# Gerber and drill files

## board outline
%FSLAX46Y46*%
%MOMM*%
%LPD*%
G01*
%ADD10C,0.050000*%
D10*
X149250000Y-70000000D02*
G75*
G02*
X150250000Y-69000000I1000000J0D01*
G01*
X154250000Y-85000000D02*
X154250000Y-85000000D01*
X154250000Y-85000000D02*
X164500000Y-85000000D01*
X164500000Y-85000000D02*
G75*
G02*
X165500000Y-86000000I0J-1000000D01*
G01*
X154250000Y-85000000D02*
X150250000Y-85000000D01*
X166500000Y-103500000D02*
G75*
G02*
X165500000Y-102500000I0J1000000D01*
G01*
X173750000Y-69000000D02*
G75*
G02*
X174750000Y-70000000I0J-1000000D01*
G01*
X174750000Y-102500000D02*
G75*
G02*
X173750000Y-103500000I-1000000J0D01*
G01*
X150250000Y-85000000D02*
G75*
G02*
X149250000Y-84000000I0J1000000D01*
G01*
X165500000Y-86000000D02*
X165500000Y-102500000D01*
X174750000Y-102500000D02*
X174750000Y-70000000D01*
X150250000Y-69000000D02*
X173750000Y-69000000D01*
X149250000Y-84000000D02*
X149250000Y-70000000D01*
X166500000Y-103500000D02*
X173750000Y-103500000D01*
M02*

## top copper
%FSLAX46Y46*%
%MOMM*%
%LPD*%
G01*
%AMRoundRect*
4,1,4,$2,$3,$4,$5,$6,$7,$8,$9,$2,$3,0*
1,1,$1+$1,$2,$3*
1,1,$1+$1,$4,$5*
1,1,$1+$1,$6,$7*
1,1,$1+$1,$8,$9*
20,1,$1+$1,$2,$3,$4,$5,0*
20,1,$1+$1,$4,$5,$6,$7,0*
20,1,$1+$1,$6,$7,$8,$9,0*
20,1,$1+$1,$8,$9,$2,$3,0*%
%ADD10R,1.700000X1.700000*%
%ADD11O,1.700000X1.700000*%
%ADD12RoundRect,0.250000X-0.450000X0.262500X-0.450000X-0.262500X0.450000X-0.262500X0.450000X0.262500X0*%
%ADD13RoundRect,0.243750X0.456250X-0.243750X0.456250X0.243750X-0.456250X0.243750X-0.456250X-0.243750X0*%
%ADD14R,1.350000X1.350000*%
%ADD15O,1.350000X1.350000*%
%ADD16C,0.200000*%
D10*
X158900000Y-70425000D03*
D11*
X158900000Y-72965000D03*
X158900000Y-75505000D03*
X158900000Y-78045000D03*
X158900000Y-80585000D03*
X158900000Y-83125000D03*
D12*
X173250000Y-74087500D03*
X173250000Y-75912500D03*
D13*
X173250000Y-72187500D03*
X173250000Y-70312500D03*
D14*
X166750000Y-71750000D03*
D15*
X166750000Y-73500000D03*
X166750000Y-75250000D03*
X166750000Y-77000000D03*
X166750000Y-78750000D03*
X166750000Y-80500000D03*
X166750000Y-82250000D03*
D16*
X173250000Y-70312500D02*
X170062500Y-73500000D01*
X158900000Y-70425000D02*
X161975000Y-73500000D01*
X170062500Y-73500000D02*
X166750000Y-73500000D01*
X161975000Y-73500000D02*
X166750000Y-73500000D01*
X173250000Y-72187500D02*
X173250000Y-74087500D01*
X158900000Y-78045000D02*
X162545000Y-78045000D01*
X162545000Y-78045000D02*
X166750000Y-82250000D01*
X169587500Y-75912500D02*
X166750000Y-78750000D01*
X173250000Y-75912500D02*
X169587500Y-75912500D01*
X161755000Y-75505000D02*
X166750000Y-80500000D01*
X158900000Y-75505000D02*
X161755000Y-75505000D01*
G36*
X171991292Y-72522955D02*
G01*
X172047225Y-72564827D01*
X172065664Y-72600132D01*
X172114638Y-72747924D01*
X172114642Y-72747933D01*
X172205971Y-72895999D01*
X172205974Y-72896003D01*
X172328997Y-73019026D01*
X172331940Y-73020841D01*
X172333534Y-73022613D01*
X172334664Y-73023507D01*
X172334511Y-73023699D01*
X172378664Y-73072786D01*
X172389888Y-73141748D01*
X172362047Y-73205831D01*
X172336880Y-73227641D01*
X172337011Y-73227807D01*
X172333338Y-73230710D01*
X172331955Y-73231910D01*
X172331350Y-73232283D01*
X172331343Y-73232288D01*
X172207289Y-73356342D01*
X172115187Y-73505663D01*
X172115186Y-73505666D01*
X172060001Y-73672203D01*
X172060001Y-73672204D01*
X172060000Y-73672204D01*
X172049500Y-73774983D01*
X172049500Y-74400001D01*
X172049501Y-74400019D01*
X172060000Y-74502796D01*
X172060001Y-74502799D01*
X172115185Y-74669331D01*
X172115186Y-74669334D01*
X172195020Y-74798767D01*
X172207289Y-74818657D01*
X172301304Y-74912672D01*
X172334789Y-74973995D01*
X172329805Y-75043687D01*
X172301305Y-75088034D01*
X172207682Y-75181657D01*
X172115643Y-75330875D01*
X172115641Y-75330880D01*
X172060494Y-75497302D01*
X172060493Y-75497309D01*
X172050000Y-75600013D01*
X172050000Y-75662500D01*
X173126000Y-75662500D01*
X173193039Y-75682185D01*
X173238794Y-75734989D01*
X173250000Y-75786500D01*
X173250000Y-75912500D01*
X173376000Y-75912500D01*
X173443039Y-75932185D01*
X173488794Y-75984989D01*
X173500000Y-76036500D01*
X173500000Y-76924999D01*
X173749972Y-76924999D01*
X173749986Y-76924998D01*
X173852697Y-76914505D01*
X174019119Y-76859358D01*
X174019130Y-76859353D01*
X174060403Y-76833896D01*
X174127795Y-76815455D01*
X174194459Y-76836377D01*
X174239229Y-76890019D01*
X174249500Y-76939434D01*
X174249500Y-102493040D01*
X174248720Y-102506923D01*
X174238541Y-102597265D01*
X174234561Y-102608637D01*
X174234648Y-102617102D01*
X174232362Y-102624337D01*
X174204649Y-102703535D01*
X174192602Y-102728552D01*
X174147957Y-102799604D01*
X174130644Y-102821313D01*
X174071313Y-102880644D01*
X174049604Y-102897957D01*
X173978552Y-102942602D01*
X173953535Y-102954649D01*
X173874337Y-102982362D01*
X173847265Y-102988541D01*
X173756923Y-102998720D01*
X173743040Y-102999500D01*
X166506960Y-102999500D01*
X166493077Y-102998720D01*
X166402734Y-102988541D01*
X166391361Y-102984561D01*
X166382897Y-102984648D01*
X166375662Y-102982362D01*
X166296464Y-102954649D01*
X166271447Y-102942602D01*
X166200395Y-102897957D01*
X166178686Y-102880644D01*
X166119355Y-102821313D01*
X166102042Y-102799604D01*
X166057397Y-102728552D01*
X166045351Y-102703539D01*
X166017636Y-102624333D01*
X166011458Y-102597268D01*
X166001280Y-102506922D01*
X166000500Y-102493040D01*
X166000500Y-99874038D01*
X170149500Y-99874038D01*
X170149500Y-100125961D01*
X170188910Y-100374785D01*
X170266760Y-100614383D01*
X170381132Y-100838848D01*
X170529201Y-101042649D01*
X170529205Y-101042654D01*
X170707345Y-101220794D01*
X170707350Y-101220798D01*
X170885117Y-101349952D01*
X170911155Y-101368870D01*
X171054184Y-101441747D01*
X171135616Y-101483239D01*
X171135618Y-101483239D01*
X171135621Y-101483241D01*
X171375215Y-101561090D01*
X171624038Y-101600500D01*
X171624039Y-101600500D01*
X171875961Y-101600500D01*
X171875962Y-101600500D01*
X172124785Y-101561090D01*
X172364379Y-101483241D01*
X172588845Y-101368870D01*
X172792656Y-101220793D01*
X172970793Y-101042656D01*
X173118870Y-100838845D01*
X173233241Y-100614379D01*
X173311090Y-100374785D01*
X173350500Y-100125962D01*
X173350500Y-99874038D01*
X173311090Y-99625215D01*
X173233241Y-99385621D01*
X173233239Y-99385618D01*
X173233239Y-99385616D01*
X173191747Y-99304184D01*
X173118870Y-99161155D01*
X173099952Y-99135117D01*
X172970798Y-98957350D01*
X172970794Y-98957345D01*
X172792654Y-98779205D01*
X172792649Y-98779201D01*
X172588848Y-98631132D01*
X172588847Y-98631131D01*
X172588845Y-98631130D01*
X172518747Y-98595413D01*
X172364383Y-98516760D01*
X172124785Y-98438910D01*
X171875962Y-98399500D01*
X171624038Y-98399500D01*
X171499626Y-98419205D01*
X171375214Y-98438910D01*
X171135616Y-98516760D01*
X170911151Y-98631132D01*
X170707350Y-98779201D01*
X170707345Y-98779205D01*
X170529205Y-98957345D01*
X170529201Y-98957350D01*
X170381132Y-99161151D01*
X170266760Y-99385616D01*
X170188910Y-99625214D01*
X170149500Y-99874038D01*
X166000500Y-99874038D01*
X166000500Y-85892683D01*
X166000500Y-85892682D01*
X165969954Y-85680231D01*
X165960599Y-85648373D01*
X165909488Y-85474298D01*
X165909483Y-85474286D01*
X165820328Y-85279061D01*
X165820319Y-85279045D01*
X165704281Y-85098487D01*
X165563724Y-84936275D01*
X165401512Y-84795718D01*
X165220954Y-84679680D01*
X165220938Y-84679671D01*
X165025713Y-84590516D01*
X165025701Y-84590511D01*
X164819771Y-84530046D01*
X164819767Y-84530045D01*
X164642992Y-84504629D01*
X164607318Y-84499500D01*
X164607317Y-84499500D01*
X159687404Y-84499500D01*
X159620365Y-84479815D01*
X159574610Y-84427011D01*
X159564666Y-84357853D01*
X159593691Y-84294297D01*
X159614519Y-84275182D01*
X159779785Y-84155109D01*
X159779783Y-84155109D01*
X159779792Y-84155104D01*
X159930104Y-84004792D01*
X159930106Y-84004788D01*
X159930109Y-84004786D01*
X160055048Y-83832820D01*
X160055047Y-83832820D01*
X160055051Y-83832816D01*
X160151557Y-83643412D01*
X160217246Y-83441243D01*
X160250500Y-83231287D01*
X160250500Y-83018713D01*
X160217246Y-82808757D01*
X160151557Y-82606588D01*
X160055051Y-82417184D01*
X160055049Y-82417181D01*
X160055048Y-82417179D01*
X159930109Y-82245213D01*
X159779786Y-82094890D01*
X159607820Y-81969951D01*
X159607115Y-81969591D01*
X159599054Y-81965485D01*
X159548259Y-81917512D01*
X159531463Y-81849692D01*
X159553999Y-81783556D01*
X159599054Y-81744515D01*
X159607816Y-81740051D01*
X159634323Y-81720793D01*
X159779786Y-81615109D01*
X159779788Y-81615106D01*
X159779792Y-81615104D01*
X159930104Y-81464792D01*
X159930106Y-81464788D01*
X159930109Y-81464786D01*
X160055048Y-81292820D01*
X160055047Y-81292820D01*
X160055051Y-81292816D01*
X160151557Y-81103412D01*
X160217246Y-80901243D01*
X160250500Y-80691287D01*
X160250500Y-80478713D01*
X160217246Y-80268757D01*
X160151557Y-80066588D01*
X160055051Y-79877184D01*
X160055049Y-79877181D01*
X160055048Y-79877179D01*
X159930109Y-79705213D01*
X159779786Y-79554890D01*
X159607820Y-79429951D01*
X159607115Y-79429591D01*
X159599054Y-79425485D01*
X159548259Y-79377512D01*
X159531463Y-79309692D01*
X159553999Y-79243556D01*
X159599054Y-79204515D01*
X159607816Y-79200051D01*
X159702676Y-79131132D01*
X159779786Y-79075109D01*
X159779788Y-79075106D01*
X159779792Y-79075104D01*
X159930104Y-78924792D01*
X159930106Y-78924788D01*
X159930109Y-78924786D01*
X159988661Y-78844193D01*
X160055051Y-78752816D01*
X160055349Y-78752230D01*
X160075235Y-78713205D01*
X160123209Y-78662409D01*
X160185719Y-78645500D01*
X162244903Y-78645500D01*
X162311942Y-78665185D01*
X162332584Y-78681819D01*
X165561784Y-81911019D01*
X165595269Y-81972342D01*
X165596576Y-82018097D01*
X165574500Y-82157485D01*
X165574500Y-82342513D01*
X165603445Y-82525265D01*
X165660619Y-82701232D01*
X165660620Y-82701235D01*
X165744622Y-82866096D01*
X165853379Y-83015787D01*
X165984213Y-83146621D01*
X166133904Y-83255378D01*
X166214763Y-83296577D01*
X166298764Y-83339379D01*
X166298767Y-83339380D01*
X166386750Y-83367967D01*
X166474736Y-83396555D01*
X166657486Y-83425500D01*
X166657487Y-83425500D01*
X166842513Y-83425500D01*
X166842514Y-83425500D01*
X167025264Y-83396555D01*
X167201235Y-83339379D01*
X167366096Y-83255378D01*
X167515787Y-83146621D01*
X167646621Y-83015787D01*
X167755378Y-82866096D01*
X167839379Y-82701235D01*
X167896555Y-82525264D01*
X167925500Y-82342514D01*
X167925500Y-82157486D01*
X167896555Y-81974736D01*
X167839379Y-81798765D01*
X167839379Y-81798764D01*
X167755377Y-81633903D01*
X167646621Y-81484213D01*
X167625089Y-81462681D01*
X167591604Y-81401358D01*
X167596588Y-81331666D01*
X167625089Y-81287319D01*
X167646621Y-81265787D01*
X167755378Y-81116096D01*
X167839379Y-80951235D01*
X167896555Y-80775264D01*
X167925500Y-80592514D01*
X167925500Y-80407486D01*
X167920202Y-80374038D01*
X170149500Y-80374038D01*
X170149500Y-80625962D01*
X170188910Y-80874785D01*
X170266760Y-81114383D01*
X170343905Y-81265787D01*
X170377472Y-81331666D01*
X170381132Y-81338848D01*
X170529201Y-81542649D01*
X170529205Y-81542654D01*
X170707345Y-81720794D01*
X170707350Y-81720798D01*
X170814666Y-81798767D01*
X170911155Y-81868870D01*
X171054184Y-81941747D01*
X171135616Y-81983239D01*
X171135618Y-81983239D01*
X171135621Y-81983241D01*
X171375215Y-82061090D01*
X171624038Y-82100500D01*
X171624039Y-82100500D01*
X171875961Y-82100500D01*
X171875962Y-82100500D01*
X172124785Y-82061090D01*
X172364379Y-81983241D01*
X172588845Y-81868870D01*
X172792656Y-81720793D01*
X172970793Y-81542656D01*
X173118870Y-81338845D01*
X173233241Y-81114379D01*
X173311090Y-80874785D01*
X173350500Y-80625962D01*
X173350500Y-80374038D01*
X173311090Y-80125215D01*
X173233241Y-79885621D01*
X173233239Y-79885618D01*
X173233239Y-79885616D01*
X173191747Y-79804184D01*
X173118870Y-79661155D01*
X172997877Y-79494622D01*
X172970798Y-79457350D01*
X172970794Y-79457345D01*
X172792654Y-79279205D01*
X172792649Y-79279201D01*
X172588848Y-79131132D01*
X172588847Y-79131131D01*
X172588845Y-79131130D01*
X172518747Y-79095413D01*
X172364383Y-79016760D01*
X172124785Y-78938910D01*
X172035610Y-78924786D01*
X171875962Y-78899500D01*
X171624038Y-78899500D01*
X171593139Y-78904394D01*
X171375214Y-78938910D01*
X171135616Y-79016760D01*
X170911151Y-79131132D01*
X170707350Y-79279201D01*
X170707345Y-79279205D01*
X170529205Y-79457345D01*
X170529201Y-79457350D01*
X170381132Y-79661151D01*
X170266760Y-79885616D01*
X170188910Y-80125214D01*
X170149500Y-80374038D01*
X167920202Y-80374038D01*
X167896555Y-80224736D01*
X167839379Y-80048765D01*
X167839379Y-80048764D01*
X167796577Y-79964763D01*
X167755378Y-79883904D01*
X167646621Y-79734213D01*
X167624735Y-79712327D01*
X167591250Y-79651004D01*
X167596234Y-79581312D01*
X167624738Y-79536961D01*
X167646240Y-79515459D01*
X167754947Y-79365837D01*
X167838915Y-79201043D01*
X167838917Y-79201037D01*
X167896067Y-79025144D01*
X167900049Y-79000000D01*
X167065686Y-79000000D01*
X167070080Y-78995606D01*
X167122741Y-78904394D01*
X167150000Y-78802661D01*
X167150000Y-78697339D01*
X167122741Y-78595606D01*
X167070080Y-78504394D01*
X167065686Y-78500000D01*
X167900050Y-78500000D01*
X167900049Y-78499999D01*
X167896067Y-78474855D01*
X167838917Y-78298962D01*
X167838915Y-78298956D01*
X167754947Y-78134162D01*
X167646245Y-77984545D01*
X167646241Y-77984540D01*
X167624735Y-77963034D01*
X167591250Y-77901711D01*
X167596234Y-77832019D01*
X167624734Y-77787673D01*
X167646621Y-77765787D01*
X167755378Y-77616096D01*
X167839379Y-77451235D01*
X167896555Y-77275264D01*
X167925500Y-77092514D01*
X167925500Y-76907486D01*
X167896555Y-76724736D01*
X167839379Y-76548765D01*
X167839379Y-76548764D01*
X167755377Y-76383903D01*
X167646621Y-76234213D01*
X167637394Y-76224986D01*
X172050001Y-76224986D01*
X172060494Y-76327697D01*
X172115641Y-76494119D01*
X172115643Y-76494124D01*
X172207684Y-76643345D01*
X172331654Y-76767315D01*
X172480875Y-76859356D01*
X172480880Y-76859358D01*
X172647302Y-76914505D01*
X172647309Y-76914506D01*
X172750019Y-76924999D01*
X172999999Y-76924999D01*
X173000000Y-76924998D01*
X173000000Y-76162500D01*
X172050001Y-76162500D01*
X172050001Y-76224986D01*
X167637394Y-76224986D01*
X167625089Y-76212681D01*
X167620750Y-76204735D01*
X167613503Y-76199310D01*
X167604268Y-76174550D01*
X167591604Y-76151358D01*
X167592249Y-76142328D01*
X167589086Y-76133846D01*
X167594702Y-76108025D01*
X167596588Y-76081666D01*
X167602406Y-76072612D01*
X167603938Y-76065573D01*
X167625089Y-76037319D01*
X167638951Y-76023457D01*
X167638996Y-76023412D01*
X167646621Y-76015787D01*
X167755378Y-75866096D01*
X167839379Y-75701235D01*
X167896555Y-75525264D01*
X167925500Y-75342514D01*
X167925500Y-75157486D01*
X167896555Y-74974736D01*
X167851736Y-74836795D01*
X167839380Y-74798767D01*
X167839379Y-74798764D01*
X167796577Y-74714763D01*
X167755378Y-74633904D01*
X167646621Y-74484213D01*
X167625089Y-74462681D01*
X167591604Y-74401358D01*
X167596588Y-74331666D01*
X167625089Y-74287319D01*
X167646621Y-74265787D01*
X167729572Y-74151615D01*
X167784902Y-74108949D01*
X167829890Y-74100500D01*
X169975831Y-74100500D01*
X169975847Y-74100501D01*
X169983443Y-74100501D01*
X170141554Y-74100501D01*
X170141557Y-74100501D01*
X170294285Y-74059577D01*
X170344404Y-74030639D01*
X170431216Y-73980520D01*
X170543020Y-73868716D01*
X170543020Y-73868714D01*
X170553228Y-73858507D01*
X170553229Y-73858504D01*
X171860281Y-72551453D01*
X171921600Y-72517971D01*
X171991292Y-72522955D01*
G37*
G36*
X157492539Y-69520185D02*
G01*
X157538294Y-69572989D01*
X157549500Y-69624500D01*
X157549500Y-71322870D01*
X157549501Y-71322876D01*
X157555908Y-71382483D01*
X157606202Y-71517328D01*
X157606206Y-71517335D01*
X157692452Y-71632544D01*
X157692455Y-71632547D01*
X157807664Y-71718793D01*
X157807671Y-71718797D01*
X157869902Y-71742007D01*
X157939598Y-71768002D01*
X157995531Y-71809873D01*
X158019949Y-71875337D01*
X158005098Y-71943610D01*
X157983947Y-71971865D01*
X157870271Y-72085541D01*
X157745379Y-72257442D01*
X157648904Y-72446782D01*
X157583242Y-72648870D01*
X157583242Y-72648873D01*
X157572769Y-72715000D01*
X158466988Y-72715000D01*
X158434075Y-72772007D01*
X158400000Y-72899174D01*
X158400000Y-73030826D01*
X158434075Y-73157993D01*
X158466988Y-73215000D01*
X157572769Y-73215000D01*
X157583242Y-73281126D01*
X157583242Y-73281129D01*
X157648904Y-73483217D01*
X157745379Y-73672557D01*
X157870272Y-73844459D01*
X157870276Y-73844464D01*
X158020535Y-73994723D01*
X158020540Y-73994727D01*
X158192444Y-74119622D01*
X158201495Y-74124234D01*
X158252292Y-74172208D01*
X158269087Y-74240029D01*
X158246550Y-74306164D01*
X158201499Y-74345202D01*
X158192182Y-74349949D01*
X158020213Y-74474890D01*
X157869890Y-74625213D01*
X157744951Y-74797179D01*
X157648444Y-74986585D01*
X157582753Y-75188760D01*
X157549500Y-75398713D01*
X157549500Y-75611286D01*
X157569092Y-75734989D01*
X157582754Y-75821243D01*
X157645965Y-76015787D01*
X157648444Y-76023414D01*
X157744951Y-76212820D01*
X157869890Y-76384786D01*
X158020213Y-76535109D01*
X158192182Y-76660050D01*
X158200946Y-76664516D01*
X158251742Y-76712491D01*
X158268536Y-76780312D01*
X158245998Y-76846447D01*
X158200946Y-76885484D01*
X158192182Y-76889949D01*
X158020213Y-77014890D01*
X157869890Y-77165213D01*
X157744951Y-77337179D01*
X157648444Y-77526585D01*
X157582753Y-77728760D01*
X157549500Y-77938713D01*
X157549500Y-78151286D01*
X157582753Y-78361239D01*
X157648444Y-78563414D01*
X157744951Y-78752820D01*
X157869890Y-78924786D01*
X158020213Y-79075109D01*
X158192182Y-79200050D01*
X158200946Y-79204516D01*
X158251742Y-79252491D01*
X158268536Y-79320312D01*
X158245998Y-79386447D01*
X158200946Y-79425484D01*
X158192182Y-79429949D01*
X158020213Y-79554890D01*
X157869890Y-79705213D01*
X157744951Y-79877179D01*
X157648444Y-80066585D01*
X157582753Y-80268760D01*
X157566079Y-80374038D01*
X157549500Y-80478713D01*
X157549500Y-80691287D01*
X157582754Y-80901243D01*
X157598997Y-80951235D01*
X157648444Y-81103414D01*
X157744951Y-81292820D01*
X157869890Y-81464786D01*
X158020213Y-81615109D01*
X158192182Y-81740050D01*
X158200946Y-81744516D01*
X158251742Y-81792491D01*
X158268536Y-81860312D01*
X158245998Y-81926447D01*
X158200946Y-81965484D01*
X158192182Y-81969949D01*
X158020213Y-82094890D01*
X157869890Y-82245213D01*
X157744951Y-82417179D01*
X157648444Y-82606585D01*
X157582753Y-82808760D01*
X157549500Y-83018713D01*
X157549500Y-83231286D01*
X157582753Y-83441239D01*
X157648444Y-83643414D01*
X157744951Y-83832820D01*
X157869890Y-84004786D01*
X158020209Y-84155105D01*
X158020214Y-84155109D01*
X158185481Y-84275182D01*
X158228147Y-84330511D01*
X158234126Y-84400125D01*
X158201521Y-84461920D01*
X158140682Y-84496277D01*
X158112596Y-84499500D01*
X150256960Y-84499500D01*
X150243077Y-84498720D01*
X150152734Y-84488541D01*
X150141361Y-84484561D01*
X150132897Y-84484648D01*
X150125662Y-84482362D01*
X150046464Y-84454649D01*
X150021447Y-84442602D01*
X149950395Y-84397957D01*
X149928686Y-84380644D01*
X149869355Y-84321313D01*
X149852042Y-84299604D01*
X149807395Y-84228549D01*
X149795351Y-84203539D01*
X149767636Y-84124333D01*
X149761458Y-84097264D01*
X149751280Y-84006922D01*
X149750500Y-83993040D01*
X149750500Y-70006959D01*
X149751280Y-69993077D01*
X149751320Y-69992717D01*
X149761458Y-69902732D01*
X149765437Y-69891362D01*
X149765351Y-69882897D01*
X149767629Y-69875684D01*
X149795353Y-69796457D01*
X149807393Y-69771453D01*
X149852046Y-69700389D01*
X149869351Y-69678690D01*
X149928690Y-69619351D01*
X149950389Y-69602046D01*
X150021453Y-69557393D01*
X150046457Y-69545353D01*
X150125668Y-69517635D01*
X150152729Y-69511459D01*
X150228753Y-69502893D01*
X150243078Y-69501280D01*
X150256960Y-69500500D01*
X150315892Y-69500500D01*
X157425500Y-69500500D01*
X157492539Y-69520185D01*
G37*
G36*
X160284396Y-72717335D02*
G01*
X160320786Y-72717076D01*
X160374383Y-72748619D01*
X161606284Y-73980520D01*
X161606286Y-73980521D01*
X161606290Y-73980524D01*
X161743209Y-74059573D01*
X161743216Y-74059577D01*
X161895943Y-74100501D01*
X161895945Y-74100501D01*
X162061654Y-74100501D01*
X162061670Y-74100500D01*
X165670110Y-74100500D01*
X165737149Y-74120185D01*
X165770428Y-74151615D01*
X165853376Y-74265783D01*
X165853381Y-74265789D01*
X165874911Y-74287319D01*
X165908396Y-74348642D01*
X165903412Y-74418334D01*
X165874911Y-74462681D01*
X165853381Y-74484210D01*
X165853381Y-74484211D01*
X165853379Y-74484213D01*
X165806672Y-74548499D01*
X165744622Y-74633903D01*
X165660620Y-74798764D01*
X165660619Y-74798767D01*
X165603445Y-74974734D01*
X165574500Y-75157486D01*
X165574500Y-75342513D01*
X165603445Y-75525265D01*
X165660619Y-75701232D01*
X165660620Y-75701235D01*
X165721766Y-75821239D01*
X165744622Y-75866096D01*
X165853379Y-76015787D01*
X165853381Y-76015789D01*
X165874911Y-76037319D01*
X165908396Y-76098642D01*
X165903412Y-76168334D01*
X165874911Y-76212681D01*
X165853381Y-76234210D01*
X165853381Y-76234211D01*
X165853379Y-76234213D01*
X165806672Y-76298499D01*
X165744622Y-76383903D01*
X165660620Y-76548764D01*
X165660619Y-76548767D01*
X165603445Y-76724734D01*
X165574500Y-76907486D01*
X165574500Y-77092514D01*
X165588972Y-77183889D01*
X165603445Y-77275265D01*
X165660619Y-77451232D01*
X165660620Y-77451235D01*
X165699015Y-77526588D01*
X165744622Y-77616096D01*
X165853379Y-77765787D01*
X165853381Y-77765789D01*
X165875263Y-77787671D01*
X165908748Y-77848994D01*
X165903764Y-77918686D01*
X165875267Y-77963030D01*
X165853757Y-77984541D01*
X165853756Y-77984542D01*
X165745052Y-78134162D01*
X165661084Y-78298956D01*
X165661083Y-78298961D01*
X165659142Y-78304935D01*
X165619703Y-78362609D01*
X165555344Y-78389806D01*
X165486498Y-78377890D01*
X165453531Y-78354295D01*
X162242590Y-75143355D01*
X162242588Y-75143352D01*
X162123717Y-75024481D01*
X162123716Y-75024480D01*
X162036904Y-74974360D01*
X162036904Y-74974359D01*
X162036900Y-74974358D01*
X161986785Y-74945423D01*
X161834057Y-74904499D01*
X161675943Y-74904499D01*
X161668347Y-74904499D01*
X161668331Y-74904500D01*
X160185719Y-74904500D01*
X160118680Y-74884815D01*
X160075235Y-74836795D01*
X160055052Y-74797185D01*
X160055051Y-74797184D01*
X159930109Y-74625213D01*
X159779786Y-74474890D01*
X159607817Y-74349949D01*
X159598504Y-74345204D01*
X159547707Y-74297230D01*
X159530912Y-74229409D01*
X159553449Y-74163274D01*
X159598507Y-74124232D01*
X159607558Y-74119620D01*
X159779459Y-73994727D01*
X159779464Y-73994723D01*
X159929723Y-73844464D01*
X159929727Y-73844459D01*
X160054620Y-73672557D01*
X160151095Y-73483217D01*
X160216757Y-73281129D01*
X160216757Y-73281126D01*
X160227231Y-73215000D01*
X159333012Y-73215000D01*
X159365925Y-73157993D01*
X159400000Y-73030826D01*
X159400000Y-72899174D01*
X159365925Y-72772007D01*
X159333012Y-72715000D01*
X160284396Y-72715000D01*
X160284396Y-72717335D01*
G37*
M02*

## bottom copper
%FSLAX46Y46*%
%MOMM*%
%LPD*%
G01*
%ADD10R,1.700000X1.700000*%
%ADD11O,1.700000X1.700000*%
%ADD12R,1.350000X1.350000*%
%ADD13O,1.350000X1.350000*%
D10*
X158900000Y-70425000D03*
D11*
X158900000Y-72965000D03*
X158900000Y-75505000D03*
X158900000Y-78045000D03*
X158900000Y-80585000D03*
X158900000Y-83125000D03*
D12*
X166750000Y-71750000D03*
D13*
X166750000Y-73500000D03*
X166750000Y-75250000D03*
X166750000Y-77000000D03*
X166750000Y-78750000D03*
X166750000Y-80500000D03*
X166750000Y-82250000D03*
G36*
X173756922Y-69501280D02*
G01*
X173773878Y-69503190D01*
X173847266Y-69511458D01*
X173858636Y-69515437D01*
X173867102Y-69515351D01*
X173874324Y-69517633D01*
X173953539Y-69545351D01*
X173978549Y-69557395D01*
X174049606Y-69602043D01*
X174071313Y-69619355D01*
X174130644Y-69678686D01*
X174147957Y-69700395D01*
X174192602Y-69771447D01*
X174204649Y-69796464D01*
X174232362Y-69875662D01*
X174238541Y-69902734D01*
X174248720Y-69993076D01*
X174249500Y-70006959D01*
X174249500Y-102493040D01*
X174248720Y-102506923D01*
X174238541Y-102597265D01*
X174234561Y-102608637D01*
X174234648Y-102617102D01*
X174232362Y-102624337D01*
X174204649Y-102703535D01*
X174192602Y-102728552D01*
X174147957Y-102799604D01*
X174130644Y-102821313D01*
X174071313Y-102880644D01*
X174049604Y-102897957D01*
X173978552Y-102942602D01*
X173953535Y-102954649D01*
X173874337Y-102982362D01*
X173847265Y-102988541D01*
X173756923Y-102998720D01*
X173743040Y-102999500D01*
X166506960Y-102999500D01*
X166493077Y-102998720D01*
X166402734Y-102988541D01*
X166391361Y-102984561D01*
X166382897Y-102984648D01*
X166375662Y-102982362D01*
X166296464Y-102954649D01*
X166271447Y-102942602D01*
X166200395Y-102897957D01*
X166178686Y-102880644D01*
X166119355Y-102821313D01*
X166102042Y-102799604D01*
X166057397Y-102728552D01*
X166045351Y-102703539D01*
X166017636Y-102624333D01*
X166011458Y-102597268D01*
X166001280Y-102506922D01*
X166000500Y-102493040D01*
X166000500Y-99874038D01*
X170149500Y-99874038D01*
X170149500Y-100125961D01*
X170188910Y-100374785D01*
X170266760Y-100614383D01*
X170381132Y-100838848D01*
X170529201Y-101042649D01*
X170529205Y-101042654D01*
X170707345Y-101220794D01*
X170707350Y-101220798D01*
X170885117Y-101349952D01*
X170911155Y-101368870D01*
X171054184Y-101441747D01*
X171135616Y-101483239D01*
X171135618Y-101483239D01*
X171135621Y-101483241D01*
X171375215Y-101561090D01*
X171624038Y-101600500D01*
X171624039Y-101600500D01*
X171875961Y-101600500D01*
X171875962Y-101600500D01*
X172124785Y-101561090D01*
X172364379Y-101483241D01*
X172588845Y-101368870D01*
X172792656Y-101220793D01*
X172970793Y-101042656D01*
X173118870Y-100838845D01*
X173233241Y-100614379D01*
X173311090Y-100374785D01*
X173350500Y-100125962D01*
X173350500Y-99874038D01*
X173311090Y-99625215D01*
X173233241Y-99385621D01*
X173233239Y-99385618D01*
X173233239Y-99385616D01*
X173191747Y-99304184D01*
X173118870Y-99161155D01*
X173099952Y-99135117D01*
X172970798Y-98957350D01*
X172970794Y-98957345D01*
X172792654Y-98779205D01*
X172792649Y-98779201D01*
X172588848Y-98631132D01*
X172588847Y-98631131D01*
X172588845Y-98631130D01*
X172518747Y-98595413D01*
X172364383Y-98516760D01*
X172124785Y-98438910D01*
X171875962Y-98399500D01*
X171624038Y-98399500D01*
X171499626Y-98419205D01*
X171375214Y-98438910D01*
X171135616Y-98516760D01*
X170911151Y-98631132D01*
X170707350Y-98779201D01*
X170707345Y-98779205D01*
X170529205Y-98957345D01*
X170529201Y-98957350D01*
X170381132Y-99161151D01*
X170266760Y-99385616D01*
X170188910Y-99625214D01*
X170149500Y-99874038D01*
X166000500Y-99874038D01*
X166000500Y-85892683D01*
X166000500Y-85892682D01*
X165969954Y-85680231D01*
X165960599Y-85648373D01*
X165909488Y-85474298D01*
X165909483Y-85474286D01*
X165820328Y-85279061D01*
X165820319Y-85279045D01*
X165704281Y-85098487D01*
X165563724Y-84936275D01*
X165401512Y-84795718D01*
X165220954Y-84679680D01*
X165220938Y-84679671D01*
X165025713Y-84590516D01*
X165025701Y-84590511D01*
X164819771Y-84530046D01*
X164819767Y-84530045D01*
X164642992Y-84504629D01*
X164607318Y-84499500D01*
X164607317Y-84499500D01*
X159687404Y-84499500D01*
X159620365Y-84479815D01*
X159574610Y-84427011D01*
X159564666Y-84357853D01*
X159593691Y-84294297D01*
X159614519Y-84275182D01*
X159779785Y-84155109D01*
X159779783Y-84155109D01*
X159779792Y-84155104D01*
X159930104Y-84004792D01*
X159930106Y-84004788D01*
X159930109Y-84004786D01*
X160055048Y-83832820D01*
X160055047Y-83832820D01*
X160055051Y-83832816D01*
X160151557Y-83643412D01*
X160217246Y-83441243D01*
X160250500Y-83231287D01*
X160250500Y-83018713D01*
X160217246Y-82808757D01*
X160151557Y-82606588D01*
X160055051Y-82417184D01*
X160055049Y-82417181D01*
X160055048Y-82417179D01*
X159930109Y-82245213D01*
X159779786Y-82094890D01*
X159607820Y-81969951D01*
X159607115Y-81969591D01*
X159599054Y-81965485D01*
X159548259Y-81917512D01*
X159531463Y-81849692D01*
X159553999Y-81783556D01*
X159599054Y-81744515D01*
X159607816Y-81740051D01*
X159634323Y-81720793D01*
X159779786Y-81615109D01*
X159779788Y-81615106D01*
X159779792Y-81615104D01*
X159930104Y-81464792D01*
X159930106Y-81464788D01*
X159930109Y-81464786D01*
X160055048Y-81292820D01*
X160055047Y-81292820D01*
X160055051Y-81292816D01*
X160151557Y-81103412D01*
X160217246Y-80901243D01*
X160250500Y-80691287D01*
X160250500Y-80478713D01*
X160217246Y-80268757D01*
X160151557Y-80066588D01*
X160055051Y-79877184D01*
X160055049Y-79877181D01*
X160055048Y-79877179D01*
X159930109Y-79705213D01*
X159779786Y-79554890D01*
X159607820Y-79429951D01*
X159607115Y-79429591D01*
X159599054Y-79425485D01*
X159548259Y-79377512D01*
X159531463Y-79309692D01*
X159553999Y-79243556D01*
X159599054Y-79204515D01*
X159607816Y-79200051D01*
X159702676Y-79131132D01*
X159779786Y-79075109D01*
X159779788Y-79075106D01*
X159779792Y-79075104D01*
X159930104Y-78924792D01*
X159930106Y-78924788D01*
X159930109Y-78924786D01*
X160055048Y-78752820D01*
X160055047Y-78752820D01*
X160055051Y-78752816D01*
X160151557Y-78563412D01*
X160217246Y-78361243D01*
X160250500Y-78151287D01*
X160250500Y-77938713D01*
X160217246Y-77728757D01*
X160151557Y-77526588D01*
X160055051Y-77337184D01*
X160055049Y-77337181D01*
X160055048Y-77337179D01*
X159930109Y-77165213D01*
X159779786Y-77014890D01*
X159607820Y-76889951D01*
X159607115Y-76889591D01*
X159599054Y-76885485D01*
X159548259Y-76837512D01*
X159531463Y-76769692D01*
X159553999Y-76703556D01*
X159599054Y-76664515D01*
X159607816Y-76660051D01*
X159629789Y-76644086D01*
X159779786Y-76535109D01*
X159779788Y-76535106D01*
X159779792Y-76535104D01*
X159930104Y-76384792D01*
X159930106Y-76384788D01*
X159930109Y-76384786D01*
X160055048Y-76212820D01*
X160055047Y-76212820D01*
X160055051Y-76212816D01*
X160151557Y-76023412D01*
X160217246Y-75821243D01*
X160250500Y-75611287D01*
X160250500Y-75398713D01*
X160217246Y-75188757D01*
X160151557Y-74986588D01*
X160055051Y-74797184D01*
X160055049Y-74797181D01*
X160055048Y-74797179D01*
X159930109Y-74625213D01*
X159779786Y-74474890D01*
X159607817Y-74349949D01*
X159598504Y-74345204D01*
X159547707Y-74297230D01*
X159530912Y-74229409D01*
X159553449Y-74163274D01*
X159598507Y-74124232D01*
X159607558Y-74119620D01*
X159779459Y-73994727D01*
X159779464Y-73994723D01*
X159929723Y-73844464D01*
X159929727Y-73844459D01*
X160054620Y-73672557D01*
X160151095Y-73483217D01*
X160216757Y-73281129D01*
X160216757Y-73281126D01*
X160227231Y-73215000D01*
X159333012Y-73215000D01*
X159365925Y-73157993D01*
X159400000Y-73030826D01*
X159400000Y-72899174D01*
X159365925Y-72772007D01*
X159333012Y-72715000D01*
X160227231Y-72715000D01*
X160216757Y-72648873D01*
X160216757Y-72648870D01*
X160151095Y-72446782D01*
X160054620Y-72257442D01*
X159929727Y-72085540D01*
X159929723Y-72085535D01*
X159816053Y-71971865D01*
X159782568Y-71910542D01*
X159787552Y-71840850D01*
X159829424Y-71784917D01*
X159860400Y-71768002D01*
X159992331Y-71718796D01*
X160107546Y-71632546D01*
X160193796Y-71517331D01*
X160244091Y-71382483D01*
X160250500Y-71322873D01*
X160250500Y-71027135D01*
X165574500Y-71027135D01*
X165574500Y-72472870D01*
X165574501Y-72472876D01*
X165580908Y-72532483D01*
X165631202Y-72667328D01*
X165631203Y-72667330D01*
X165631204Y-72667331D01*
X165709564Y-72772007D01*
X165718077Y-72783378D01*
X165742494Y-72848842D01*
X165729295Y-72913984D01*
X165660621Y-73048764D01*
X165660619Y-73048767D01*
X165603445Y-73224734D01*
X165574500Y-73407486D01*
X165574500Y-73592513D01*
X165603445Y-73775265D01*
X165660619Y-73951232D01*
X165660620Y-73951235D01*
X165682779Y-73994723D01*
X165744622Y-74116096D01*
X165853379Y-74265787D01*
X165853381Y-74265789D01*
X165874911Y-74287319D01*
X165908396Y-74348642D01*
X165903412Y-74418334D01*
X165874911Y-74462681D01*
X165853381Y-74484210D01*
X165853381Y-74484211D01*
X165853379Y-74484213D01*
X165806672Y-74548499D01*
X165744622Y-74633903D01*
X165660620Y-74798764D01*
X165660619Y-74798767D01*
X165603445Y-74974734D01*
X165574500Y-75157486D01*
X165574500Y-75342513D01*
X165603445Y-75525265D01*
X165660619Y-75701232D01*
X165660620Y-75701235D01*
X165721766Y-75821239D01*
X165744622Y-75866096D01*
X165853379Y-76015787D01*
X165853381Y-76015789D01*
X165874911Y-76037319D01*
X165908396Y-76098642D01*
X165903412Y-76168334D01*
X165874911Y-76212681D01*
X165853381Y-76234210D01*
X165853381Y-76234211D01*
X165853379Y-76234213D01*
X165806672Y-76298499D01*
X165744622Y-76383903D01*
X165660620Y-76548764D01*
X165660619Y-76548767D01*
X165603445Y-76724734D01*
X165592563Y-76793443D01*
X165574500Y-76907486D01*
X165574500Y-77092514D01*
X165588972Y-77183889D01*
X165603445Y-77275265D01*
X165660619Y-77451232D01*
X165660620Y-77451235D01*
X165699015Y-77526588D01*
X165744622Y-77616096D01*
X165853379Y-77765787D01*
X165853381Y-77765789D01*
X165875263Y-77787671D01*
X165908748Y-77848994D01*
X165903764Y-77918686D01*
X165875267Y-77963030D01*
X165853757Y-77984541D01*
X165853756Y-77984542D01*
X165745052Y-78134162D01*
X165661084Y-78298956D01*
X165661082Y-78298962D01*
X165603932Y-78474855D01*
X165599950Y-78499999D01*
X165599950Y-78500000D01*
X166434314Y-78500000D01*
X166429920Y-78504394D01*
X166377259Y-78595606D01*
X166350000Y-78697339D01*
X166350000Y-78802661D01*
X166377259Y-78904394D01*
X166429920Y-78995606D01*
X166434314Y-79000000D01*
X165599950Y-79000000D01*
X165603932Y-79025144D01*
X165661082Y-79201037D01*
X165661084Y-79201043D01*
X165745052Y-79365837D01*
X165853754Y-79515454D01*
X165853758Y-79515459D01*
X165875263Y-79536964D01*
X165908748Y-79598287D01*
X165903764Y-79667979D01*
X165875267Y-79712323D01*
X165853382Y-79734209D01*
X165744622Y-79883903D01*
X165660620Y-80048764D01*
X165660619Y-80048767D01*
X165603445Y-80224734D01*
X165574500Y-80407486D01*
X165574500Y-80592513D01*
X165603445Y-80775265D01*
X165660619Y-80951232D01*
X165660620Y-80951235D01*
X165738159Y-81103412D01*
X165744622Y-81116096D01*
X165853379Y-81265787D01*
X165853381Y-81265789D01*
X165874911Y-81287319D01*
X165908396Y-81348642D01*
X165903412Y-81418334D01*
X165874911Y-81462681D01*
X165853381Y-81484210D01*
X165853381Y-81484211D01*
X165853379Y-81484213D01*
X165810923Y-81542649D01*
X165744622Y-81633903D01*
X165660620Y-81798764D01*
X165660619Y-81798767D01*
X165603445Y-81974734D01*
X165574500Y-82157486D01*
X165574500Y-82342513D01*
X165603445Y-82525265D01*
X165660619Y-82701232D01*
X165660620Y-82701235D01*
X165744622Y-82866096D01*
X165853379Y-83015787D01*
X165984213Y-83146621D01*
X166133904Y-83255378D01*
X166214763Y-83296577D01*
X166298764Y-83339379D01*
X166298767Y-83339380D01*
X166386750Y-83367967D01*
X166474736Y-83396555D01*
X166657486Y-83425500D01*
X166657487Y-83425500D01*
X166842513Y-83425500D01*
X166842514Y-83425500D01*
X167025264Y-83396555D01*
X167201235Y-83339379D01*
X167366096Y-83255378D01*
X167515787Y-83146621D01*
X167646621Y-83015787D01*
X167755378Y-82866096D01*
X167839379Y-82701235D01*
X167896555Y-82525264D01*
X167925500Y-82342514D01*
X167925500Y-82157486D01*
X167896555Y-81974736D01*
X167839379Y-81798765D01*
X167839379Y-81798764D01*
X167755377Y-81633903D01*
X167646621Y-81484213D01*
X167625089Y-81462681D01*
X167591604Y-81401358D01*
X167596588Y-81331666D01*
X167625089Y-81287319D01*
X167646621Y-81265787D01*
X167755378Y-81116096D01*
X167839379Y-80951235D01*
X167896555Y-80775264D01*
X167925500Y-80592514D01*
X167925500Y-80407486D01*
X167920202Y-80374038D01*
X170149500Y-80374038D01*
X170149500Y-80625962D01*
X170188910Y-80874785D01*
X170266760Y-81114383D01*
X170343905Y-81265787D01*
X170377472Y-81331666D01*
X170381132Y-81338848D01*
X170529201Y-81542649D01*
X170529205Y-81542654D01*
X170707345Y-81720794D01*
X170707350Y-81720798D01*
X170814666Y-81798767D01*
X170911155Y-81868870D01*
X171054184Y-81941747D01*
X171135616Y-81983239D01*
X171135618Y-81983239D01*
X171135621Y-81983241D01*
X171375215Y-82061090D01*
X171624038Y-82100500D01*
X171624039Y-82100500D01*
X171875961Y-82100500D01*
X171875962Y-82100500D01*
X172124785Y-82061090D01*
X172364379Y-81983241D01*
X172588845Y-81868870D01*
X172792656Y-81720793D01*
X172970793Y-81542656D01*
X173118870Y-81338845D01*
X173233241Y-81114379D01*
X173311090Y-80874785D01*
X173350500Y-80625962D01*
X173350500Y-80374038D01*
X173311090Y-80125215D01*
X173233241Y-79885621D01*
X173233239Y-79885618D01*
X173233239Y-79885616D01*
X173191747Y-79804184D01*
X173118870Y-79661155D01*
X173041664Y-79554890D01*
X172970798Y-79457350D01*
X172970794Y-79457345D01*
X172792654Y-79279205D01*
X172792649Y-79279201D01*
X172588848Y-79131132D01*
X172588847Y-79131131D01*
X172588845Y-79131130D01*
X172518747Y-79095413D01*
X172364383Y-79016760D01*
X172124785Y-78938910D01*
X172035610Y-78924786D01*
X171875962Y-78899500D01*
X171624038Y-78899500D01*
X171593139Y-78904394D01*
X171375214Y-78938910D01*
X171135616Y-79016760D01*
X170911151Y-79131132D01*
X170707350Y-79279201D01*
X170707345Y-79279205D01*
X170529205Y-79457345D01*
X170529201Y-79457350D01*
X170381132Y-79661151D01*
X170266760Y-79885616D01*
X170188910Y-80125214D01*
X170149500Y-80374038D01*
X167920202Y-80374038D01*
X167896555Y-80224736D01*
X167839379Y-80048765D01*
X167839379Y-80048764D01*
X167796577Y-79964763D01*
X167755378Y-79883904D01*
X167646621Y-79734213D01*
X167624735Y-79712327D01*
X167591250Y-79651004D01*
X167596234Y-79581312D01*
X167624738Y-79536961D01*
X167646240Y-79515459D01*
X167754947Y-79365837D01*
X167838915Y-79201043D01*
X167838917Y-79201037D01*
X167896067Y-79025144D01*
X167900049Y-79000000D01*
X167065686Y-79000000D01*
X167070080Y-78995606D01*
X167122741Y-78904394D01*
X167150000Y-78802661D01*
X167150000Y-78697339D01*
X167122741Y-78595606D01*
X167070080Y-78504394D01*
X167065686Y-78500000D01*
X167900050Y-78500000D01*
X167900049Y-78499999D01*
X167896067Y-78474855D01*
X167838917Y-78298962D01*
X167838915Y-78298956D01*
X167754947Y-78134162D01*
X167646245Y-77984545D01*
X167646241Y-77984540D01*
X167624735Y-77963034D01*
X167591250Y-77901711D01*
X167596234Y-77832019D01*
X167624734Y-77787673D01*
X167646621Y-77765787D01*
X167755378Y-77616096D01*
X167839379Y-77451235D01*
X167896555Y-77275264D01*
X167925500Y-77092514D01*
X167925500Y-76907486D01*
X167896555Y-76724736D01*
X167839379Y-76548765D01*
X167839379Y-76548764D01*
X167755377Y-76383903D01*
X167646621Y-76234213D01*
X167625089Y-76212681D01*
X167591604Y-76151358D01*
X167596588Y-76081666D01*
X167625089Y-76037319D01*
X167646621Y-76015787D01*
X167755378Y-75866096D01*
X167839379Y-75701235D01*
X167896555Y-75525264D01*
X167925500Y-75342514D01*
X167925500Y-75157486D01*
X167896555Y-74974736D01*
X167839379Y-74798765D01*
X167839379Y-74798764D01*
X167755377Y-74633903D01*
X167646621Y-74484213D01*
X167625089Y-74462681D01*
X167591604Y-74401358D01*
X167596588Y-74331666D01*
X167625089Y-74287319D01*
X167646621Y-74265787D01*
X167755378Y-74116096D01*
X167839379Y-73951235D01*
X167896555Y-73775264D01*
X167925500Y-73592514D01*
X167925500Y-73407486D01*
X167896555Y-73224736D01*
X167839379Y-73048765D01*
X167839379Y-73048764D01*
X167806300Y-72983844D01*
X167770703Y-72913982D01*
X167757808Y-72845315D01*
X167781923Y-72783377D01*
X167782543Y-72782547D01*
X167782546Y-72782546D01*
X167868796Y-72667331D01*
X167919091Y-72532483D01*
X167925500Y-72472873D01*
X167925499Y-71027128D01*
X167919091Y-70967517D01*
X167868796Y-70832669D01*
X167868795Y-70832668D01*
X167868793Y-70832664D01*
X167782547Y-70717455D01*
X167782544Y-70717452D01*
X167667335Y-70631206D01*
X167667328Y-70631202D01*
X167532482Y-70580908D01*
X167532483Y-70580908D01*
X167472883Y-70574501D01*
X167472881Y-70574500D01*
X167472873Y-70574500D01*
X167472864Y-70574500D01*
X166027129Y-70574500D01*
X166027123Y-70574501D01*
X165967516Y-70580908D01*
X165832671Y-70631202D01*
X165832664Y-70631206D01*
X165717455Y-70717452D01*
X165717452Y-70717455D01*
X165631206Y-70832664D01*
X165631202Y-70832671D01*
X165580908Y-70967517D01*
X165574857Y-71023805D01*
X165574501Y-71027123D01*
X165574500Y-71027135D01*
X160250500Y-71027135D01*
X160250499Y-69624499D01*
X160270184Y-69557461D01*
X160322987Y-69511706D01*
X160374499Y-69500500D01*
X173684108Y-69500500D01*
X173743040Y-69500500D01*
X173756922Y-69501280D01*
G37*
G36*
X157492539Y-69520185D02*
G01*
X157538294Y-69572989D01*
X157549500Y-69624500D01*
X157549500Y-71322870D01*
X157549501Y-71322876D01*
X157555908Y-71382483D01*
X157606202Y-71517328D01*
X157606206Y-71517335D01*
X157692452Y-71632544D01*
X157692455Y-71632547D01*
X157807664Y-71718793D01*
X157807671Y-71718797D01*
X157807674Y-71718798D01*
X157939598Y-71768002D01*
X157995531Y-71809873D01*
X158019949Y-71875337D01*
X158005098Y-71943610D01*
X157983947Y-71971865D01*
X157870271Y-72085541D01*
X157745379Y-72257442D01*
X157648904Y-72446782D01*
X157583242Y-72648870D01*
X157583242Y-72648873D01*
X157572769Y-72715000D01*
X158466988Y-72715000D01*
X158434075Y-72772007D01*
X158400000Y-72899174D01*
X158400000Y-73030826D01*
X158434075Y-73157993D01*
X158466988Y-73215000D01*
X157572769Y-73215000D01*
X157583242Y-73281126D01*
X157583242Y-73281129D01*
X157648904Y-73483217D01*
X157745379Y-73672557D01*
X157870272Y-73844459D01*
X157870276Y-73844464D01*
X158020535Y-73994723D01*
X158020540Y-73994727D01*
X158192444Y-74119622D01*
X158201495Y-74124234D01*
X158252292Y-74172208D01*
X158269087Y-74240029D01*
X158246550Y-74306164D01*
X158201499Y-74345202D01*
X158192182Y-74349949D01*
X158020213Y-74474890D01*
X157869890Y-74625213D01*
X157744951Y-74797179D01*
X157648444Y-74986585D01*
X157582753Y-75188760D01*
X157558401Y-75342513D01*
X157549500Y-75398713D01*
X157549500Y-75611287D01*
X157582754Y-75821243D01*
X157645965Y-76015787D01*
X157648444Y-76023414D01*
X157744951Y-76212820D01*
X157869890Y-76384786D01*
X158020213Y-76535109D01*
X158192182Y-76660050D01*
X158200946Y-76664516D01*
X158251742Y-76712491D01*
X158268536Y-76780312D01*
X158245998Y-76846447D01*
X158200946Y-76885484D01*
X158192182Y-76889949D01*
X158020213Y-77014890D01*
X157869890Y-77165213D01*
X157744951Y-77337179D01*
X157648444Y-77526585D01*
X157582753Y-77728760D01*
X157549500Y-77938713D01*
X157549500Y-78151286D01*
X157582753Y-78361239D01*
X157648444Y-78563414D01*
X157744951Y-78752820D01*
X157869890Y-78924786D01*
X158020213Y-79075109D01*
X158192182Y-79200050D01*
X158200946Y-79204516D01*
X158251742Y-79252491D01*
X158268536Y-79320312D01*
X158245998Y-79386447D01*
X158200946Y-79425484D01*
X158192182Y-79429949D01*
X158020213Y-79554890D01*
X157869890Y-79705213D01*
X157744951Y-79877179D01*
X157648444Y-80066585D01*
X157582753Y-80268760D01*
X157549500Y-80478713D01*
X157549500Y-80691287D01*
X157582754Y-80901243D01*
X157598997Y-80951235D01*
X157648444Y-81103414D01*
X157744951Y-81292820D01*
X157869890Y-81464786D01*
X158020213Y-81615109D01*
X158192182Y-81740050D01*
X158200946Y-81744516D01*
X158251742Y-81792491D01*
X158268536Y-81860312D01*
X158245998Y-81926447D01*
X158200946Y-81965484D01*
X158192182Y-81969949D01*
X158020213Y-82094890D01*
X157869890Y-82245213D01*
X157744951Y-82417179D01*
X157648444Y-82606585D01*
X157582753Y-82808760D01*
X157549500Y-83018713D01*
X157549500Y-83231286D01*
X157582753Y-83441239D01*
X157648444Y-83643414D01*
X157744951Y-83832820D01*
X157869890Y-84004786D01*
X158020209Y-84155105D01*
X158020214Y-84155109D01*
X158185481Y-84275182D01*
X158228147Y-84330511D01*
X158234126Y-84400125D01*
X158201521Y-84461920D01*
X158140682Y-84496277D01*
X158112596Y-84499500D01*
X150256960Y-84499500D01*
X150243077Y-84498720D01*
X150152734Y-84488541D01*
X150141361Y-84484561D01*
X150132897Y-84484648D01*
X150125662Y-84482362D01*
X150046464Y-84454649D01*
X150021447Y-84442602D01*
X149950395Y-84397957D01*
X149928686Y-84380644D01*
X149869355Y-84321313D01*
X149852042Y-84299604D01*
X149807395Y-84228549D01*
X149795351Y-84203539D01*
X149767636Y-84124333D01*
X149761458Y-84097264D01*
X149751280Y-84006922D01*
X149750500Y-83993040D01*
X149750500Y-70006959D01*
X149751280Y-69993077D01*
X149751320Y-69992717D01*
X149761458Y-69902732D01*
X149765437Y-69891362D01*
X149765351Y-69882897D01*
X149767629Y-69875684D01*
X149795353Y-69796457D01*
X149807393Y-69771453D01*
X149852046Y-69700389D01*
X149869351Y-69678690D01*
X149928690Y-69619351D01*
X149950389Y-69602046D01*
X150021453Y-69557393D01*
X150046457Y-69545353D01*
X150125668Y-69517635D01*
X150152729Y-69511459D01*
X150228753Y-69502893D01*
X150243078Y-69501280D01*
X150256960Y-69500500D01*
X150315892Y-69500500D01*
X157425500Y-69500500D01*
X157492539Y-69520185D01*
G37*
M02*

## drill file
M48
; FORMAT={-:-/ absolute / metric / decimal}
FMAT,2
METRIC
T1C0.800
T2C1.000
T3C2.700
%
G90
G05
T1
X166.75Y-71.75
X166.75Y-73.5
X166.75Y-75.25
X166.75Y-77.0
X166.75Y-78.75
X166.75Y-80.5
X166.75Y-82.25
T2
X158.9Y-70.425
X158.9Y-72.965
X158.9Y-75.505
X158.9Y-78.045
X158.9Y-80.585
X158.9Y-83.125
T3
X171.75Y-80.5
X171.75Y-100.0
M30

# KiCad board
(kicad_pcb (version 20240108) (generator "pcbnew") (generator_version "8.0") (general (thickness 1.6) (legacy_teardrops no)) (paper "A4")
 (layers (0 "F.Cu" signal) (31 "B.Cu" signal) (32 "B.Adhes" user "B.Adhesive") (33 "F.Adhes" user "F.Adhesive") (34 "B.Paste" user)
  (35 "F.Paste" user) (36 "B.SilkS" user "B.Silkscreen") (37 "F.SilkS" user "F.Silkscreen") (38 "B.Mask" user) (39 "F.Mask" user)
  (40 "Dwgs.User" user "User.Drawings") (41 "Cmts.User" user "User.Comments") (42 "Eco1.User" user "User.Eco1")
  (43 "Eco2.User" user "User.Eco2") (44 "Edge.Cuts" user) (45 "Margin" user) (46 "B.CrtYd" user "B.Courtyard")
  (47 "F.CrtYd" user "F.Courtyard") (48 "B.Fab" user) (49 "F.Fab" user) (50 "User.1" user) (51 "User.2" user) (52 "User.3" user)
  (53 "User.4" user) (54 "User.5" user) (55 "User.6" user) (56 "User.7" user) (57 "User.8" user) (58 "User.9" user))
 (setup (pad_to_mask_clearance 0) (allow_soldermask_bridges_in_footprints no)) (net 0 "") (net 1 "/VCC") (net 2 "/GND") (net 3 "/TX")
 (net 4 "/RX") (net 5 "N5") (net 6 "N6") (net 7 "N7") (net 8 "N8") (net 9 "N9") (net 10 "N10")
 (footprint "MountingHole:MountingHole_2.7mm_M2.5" (layer "F.Cu") (at 171.75 100)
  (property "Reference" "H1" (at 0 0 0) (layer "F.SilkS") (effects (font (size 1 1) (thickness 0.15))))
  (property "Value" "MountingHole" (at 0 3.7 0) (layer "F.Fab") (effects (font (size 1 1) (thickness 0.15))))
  (pad "" np_thru_hole circle (at 0 0) (size 2.7 2.7) (drill 2.7) (layers "*.Cu" "*.Mask")))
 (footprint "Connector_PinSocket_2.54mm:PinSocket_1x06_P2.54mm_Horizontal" (layer "F.Cu") (at 158.9 70.425)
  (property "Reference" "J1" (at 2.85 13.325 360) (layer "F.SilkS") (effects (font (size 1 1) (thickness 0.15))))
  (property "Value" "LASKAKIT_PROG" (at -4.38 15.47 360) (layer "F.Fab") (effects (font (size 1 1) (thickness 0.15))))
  (pad "1" thru_hole rect (at 0 0) (size 1.7 1.7) (drill 1) (layers "*.Cu" "*.Mask") (remove_unused_layers no) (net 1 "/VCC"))
  (pad "2" thru_hole oval (at 0 2.54) (size 1.7 1.7) (drill 1) (layers "*.Cu" "*.Mask") (remove_unused_layers no) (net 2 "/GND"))
  (pad "3" thru_hole oval (at 0 5.08) (size 1.7 1.7) (drill 1) (layers "*.Cu" "*.Mask") (remove_unused_layers no) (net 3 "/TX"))
  (pad "4" thru_hole oval (at 0 7.62) (size 1.7 1.7) (drill 1) (layers "*.Cu" "*.Mask") (remove_unused_layers no) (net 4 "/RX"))
  (pad "5" thru_hole oval (at 0 10.16) (size 1.7 1.7) (drill 1) (layers "*.Cu" "*.Mask") (remove_unused_layers no) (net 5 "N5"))
  (pad "6" thru_hole oval (at 0 12.7) (size 1.7 1.7) (drill 1) (layers "*.Cu" "*.Mask") (remove_unused_layers no) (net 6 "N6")))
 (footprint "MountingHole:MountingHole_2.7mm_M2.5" (layer "F.Cu") (at 171.75 80.5)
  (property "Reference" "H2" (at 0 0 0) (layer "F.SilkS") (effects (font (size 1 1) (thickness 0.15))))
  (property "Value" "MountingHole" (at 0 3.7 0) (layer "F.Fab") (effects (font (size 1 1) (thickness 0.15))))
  (pad "" np_thru_hole circle (at 0 0) (size 2.7 2.7) (drill 2.7) (layers "*.Cu" "*.Mask")))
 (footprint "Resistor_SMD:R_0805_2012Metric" (layer "F.Cu") (at 173.25 75 -90)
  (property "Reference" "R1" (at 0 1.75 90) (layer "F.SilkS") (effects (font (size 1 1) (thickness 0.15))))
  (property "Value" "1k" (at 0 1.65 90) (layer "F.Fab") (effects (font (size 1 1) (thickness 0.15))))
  (pad "1" smd roundrect (at -0.9125 0 270) (size 1.025 1.4) (layers "F.Cu" "F.Paste" "F.Mask") (roundrect_rratio 0.243902) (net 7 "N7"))
  (pad "2" smd roundrect (at 0.9125 0 270) (size 1.025 1.4) (layers "F.Cu" "F.Paste" "F.Mask") (roundrect_rratio 0.243902) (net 2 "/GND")))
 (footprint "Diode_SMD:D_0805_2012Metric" (layer "F.Cu") (at 173.25 71.25 90)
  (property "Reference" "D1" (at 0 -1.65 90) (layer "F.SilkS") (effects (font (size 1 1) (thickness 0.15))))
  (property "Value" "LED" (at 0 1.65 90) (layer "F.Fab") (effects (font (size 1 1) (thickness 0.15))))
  (pad "1" smd roundrect (at -0.9375 0 90) (size 0.975 1.4) (layers "F.Cu" "F.Paste" "F.Mask") (roundrect_rratio 0.25) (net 7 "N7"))
  (pad "2" smd roundrect (at 0.9375 0 90) (size 0.975 1.4) (layers "F.Cu" "F.Paste" "F.Mask") (roundrect_rratio 0.25) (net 1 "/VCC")))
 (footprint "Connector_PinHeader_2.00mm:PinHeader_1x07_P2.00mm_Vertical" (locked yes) (layer "F.Cu") (at 166.75 71.75)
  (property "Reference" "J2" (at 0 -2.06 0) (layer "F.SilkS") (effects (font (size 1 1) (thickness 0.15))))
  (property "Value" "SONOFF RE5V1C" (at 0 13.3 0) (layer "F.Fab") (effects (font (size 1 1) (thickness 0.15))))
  (pad "1" thru_hole rect (at 0 0) (size 1.35 1.35) (drill 0.8) (layers "*.Cu" "*.Mask") (remove_unused_layers no) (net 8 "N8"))
  (pad "2" thru_hole oval (at 0 1.75) (size 1.35 1.35) (drill 0.8) (layers "*.Cu" "*.Mask") (remove_unused_layers no) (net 1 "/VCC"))
  (pad "3" thru_hole oval (at 0 3.5) (size 1.35 1.35) (drill 0.8) (layers "*.Cu" "*.Mask") (remove_unused_layers no) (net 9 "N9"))
  (pad "4" thru_hole oval (at 0 5.25) (size 1.35 1.35) (drill 0.8) (layers "*.Cu" "*.Mask") (remove_unused_layers no) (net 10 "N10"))
  (pad "5" thru_hole oval (at 0 7) (size 1.35 1.35) (drill 0.8) (layers "*.Cu" "*.Mask") (remove_unused_layers no) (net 2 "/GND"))
  (pad "6" thru_hole oval (at 0 8.75) (size 1.35 1.35) (drill 0.8) (layers "*.Cu" "*.Mask") (remove_unused_layers no) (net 3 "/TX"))
  (pad "7" thru_hole oval (at 0 10.5) (size 1.35 1.35) (drill 0.8) (layers "*.Cu" "*.Mask") (remove_unused_layers no) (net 4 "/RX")))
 (gr_arc (start 149.25 70) (mid 149.542893 69.292893) (end 150.25 69) (stroke (width 0.05) (type default)) (layer "Edge.Cuts"))
 (gr_line (start 154.25 85) (end 154.25 85) (stroke (width 0.05) (type default)) (layer "Edge.Cuts"))
 (gr_line (start 154.25 85) (end 164.5 85) (stroke (width 0.05) (type default)) (layer "Edge.Cuts"))
 (gr_arc (start 164.5 85) (mid 165.207107 85.292893) (end 165.5 86) (stroke (width 0.05) (type default)) (layer "Edge.Cuts"))
 (gr_line (start 154.25 85) (end 150.25 85) (stroke (width 0.05) (type default)) (layer "Edge.Cuts"))
 (gr_arc (start 166.5 103.5) (mid 165.792893 103.207107) (end 165.5 102.5) (stroke (width 0.05) (type default)) (layer "Edge.Cuts"))
 (gr_arc (start 173.75 69) (mid 174.457107 69.292893) (end 174.75 70) (stroke (width 0.05) (type default)) (layer "Edge.Cuts"))
 (gr_arc (start 174.75 102.5) (mid 174.457107 103.207107) (end 173.75 103.5) (stroke (width 0.05) (type default)) (layer "Edge.Cuts"))
 (gr_arc (start 150.25 85) (mid 149.542893 84.707107) (end 149.25 84) (stroke (width 0.05) (type default)) (layer "Edge.Cuts"))
 (gr_line (start 165.5 86) (end 165.5 102.5) (stroke (width 0.05) (type default)) (layer "Edge.Cuts"))
 (gr_line (start 174.75 102.5) (end 174.75 70) (stroke (width 0.05) (type default)) (layer "Edge.Cuts"))
 (gr_line (start 150.25 69) (end 173.75 69) (stroke (width 0.05) (type default)) (layer "Edge.Cuts"))
 (gr_line (start 149.25 84) (end 149.25 70) (stroke (width 0.05) (type default)) (layer "Edge.Cuts"))
 (gr_line (start 166.5 103.5) (end 173.75 103.5) (stroke (width 0.05) (type default)) (layer "Edge.Cuts"))
 (segment (start 173.25 70.3125) (end 170.0625 73.5) (width 0.2) (layer "F.Cu") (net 1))
 (segment (start 158.9 70.425) (end 161.975 73.5) (width 0.2) (layer "F.Cu") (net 1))
 (segment (start 170.0625 73.5) (end 166.75 73.5) (width 0.2) (layer "F.Cu") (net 1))
 (segment (start 161.975 73.5) (end 166.75 73.5) (width 0.2) (layer "F.Cu") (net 1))
 (segment (start 173.25 72.1875) (end 173.25 74.0875) (width 0.2) (layer "F.Cu") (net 7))
 (segment (start 158.9 78.045) (end 162.545 78.045) (width 0.2) (layer "F.Cu") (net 4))
 (segment (start 162.545 78.045) (end 166.75 82.25) (width 0.2) (layer "F.Cu") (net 4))
 (segment (start 169.5875 75.9125) (end 166.75 78.75) (width 0.2) (layer "F.Cu") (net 2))
 (segment (start 173.25 75.9125) (end 169.5875 75.9125) (width 0.2) (layer "F.Cu") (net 2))
 (segment (start 161.755 75.505) (end 166.75 80.5) (width 0.2) (layer "F.Cu") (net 3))
 (segment (start 158.9 75.505) (end 161.755 75.505) (width 0.2) (layer "F.Cu") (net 3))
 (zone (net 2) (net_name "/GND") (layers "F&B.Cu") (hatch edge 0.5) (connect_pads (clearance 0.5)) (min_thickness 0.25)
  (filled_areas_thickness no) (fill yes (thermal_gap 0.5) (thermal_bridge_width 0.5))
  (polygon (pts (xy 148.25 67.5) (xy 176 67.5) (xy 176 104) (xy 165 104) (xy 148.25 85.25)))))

